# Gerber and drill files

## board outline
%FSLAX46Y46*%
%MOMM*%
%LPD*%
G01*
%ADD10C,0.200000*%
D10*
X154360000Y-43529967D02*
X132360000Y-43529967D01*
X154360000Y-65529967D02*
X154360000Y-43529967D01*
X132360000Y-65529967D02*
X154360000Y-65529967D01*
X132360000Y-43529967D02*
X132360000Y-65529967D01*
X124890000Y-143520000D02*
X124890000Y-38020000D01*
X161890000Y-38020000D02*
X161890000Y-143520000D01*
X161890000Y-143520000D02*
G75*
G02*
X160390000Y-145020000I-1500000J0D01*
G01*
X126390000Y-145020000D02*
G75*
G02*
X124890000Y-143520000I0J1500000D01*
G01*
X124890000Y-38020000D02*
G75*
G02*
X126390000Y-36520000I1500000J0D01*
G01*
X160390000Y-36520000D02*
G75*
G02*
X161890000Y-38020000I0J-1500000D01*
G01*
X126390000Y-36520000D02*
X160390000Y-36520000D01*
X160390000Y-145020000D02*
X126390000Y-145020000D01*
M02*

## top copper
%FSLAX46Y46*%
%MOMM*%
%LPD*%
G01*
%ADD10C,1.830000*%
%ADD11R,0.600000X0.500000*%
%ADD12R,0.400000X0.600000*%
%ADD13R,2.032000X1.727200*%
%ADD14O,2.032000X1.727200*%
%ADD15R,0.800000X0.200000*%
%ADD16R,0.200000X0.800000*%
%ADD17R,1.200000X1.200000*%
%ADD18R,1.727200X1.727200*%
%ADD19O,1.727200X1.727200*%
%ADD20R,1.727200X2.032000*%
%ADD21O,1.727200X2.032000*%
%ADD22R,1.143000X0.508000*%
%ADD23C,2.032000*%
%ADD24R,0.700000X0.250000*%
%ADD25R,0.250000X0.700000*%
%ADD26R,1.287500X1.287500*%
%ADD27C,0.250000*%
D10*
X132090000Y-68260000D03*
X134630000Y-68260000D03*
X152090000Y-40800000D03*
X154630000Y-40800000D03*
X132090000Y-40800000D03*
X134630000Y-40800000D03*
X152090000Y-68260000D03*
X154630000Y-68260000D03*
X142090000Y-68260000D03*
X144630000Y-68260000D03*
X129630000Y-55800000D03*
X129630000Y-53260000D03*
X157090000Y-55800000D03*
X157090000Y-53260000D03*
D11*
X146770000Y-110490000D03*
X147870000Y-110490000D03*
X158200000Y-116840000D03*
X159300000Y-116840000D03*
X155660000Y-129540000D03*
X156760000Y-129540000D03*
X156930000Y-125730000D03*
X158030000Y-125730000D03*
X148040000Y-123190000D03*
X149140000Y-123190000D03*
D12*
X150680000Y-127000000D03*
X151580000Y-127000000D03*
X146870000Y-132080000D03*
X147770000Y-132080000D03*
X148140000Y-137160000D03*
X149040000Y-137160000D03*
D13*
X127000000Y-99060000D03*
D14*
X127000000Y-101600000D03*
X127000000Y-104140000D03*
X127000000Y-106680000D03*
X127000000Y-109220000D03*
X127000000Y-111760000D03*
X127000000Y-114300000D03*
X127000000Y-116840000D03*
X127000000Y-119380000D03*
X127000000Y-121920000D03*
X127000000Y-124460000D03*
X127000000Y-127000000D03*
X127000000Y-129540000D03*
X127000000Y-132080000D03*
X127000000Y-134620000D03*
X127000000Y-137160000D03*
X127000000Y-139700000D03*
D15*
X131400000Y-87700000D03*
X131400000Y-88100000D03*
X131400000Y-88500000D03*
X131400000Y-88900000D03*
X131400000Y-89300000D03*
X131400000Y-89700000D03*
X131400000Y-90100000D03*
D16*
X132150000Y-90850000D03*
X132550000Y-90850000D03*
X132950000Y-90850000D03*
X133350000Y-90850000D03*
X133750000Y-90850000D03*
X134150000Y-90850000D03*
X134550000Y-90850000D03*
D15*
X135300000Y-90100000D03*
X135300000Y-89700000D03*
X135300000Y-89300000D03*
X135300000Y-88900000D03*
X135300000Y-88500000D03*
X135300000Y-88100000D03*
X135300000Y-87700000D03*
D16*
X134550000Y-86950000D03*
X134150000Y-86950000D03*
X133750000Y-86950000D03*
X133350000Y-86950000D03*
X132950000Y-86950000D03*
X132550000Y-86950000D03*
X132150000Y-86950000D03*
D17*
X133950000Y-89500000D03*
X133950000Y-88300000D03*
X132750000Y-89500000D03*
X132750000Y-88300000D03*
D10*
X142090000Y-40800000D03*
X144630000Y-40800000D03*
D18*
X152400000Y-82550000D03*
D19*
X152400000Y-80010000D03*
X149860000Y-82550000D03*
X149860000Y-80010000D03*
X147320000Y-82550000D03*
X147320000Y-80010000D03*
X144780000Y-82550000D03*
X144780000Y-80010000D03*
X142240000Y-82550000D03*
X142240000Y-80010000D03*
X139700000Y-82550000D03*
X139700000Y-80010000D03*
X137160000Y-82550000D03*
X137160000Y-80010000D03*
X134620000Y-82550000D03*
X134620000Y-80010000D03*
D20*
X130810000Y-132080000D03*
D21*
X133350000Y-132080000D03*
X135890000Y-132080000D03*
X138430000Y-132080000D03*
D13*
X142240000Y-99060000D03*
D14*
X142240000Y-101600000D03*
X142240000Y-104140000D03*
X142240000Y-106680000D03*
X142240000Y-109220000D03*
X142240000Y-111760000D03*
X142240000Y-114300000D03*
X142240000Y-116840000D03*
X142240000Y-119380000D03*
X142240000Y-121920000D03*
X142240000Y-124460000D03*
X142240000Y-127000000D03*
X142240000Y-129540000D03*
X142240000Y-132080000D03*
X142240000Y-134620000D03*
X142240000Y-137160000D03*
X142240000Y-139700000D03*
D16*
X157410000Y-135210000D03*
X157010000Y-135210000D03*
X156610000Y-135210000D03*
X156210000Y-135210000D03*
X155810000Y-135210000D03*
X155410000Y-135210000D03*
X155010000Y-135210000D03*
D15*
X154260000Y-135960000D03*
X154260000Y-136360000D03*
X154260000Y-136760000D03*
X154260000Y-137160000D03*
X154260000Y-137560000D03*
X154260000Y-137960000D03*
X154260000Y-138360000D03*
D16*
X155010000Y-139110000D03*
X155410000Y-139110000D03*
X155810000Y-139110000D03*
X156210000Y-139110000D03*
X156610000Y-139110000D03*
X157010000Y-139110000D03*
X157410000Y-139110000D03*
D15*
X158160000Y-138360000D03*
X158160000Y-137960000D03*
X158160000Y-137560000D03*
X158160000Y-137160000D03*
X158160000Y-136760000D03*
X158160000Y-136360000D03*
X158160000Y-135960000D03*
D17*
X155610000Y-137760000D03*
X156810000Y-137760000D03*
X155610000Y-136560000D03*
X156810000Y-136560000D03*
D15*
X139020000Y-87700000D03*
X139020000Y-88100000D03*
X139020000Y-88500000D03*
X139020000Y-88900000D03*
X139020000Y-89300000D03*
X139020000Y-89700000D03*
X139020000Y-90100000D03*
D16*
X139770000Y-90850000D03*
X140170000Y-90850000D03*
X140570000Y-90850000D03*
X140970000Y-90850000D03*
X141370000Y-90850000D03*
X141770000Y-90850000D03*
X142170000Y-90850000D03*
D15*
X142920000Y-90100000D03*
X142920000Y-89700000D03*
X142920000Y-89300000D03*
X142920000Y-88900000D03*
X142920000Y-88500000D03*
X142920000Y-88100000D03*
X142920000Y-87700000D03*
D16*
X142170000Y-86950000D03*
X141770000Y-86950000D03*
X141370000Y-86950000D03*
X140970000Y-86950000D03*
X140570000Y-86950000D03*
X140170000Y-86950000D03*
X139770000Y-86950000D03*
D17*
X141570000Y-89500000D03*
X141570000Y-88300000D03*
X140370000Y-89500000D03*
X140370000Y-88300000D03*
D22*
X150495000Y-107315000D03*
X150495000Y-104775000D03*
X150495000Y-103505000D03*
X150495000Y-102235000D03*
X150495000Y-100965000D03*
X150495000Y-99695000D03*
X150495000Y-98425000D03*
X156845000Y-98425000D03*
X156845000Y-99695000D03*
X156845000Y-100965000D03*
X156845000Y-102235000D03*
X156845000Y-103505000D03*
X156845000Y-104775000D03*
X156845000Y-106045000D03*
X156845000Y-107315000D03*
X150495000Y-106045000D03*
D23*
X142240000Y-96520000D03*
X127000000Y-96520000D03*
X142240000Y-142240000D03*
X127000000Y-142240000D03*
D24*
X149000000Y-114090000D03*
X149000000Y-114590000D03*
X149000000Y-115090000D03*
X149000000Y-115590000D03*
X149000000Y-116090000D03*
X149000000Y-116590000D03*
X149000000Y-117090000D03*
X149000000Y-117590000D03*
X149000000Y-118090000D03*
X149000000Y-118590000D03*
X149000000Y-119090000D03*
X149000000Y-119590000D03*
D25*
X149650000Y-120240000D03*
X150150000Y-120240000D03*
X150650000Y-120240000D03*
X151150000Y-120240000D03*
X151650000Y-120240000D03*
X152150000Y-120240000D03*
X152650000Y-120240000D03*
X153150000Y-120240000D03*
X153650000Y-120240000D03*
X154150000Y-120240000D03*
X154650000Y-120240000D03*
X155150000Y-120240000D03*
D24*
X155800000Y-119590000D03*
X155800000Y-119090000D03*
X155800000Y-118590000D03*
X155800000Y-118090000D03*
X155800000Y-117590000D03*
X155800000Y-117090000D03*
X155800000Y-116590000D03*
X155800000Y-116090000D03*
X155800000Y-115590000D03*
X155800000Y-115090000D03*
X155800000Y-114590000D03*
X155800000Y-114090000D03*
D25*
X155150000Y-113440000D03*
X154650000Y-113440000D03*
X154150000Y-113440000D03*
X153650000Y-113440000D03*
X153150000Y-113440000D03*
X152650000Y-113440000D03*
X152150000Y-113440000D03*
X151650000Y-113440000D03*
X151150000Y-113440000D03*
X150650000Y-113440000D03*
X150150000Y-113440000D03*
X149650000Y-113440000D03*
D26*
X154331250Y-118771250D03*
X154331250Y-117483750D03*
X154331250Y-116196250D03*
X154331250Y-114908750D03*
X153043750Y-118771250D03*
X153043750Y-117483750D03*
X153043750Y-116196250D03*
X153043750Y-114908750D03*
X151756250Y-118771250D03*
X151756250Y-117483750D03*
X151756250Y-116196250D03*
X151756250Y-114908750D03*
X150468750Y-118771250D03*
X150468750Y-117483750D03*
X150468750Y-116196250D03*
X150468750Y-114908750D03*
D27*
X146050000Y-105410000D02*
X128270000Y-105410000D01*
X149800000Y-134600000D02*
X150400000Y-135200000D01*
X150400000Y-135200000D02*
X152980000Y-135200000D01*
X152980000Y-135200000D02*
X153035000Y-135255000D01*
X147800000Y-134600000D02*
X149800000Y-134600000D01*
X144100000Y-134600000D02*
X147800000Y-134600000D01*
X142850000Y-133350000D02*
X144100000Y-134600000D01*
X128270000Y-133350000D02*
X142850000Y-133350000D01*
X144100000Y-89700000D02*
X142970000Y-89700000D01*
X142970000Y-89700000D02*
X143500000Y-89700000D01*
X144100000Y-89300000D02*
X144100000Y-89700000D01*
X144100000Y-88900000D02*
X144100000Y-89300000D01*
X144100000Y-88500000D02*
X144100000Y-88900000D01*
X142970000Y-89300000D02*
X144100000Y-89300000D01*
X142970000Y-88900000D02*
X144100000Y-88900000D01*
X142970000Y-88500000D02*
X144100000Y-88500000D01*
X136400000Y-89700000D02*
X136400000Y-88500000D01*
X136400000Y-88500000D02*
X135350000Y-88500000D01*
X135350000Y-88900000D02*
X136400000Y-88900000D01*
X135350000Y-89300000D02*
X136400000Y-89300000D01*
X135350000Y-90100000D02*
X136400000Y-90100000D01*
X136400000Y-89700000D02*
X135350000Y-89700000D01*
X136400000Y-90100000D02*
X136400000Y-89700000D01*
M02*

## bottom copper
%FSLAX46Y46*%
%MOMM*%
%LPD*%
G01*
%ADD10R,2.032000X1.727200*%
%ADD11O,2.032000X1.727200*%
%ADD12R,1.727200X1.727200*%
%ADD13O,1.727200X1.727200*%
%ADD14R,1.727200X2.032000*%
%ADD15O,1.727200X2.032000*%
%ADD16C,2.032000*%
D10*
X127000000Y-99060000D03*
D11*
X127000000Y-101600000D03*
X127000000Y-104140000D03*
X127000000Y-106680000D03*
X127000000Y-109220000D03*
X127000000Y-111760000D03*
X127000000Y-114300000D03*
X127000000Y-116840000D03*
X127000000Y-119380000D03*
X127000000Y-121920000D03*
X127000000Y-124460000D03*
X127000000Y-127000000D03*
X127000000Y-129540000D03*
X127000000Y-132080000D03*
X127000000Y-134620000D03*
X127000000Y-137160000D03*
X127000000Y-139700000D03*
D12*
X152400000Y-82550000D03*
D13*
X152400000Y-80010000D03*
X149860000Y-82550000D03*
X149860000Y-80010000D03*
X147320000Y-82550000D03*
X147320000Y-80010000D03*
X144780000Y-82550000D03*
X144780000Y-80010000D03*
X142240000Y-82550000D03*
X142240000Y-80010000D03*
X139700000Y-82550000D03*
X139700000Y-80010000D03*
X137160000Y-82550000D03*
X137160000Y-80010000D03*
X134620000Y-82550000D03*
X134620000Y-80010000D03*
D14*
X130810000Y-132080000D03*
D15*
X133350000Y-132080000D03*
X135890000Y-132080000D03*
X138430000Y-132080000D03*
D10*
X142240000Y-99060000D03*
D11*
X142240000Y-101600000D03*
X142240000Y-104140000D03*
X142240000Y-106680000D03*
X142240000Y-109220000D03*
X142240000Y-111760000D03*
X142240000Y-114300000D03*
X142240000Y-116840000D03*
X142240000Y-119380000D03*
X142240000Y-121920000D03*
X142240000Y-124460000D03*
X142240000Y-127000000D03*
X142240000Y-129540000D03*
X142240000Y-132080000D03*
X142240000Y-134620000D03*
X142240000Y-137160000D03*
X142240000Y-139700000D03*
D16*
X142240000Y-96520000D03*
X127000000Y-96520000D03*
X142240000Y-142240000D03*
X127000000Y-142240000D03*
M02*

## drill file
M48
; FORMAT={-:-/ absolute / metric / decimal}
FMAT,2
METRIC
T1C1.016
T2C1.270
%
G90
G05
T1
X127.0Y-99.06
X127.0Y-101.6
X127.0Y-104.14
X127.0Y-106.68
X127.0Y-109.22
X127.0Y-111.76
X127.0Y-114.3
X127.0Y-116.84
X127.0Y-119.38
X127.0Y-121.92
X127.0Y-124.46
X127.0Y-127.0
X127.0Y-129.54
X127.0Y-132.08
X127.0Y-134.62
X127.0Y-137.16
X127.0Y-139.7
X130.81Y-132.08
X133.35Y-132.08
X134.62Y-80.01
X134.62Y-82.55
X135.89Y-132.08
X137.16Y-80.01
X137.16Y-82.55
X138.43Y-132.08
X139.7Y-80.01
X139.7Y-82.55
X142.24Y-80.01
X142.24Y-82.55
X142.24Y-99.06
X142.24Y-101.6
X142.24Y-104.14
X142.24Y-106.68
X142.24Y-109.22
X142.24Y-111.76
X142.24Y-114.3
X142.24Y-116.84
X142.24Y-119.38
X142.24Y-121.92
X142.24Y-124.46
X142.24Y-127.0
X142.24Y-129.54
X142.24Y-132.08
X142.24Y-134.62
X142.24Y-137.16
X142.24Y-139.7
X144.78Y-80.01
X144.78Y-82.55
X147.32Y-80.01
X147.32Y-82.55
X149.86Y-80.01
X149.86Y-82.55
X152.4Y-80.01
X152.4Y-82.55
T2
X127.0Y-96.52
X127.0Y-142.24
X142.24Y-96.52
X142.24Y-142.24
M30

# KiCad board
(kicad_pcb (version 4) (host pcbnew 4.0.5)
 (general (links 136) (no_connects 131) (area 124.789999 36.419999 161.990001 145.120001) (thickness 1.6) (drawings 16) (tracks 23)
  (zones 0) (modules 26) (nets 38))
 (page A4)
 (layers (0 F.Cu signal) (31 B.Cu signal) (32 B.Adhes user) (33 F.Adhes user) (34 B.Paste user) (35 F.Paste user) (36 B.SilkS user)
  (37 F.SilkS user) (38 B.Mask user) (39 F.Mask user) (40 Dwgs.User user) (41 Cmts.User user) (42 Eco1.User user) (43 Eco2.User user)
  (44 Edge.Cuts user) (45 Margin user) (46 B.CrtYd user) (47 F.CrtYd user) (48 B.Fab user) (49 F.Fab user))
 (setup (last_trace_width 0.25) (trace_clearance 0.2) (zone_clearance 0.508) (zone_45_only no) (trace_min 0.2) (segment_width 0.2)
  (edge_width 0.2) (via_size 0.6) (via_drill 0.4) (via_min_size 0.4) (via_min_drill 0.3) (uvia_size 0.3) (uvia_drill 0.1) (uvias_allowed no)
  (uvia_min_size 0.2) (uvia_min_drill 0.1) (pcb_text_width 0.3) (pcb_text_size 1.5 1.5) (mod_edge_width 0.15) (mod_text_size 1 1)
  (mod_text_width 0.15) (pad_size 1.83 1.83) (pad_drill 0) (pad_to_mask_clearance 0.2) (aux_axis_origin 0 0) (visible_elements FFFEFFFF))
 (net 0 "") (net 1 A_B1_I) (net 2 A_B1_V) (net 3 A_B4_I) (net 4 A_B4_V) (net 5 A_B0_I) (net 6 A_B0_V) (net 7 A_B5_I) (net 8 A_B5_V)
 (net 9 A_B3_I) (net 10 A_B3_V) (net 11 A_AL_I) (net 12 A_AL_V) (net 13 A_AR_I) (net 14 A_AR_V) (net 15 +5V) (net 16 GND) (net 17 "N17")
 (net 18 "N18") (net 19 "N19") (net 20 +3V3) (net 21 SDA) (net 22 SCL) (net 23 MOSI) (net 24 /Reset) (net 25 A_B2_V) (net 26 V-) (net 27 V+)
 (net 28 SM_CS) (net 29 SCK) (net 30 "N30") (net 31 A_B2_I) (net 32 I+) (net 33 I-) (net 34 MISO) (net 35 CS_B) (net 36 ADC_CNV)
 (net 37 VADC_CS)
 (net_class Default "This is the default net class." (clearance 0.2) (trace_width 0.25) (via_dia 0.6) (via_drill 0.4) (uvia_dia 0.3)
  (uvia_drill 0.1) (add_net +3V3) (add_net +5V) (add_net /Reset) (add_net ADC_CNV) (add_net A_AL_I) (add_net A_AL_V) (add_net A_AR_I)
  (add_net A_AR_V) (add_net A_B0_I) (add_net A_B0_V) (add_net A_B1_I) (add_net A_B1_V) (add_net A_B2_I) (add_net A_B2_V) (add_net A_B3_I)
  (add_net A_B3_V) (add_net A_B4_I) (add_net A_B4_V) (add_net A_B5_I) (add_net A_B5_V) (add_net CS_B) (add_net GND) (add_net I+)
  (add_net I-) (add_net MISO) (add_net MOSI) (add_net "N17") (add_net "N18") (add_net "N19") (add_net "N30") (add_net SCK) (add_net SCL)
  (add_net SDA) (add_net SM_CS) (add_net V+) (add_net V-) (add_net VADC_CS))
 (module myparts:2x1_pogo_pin (layer F.Cu) (at 132.09 68.26)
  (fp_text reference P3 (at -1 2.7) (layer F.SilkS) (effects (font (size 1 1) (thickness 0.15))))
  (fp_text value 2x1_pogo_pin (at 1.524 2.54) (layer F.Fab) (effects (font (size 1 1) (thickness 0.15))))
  (pad 1 smd circle (at 0 0) (size 1.83 1.83) (layers F.Cu F.Paste F.Mask) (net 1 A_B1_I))
  (pad 2 smd circle (at 2.54 0) (size 1.83 1.83) (layers F.Cu F.Paste F.Mask) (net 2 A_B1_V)))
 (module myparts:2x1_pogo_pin (layer F.Cu) (at 152.09 40.8)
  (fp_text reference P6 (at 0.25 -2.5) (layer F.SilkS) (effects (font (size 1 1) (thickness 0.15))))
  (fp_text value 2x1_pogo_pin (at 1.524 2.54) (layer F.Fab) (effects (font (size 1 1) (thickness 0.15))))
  (pad 1 smd circle (at 0 0) (size 1.83 1.83) (layers F.Cu F.Paste F.Mask) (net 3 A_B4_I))
  (pad 2 smd circle (at 2.54 0) (size 1.83 1.83) (layers F.Cu F.Paste F.Mask) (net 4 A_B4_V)))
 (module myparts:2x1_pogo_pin (layer F.Cu) (at 132.09 40.8)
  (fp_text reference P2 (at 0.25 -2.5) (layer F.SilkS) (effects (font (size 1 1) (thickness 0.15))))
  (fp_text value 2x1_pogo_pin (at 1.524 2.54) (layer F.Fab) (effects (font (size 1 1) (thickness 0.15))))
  (pad 1 smd circle (at 0 0) (size 1.83 1.83) (layers F.Cu F.Paste F.Mask) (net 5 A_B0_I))
  (pad 2 smd circle (at 2.54 0) (size 1.83 1.83) (layers F.Cu F.Paste F.Mask) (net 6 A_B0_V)))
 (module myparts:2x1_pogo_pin (layer F.Cu) (at 152.09 68.26)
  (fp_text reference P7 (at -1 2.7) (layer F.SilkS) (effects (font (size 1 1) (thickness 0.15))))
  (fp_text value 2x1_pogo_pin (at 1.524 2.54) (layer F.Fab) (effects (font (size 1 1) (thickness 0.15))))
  (pad 1 smd circle (at 0 0) (size 1.83 1.83) (layers F.Cu F.Paste F.Mask) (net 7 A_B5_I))
  (pad 2 smd circle (at 2.54 0) (size 1.83 1.83) (layers F.Cu F.Paste F.Mask) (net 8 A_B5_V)))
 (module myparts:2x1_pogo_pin (layer F.Cu) (at 142.09 68.26)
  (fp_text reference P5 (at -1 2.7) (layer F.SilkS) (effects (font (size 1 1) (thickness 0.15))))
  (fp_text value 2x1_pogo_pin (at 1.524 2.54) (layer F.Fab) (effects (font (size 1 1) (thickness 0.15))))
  (pad 1 smd circle (at 0 0) (size 1.83 1.83) (layers F.Cu F.Paste F.Mask) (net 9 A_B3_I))
  (pad 2 smd circle (at 2.54 0) (size 1.83 1.83) (layers F.Cu F.Paste F.Mask) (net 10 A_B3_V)))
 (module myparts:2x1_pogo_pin (layer F.Cu) (at 129.63 55.8 90)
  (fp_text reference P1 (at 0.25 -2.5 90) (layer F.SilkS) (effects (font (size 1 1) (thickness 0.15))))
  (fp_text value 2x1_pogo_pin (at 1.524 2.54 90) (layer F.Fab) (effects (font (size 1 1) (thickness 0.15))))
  (pad 1 smd circle (at 0 0 90) (size 1.83 1.83) (layers F.Cu F.Paste F.Mask) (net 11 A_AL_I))
  (pad 2 smd circle (at 2.54 0 90) (size 1.83 1.83) (layers F.Cu F.Paste F.Mask) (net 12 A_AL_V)))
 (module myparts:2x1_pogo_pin (layer F.Cu) (at 157.09 55.8 90)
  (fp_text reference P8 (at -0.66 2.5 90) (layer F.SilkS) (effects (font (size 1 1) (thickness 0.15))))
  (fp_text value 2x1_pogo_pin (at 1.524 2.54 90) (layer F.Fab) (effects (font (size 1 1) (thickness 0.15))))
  (pad 1 smd circle (at 0 0 90) (size 1.83 1.83) (layers F.Cu F.Paste F.Mask) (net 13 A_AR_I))
  (pad 2 smd circle (at 2.54 0 90) (size 1.83 1.83) (layers F.Cu F.Paste F.Mask) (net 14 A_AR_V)))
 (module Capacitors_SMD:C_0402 (layer F.Cu) (at 147.32 110.49)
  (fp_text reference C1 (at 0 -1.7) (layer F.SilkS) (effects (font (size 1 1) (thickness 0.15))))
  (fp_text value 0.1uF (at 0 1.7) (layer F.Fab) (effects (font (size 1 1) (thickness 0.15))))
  (pad 1 smd rect (at -0.55 0) (size 0.6 0.5) (layers F.Cu F.Paste F.Mask) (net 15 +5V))
  (pad 2 smd rect (at 0.55 0) (size 0.6 0.5) (layers F.Cu F.Paste F.Mask) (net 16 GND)))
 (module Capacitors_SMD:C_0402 (layer F.Cu) (at 158.75 116.84)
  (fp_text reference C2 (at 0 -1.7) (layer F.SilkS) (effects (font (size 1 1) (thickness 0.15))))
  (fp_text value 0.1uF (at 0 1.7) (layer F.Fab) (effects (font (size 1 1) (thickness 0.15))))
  (pad 1 smd rect (at -0.55 0) (size 0.6 0.5) (layers F.Cu F.Paste F.Mask) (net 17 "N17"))
  (pad 2 smd rect (at 0.55 0) (size 0.6 0.5) (layers F.Cu F.Paste F.Mask) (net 16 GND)))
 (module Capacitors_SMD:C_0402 (layer F.Cu) (at 156.21 129.54)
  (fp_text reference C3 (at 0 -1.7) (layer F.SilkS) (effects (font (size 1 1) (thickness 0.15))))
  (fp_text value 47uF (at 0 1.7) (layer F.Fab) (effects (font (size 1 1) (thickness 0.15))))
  (pad 1 smd rect (at -0.55 0) (size 0.6 0.5) (layers F.Cu F.Paste F.Mask) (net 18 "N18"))
  (pad 2 smd rect (at 0.55 0) (size 0.6 0.5) (layers F.Cu F.Paste F.Mask) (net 16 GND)))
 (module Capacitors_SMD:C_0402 (layer F.Cu) (at 157.48 125.73)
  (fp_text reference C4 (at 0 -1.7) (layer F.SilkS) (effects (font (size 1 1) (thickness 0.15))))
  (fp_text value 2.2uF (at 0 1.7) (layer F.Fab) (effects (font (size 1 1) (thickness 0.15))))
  (pad 1 smd rect (at -0.55 0) (size 0.6 0.5) (layers F.Cu F.Paste F.Mask) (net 16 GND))
  (pad 2 smd rect (at 0.55 0) (size 0.6 0.5) (layers F.Cu F.Paste F.Mask) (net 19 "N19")))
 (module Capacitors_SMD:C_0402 (layer F.Cu) (at 148.59 123.19)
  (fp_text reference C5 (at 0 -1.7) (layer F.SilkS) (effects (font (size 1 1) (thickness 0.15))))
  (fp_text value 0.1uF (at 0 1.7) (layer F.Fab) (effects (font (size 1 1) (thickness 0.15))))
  (pad 1 smd rect (at -0.55 0) (size 0.6 0.5) (layers F.Cu F.Paste F.Mask) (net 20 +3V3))
  (pad 2 smd rect (at 0.55 0) (size 0.6 0.5) (layers F.Cu F.Paste F.Mask) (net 16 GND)))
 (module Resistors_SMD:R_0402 (layer F.Cu) (at 151.13 127)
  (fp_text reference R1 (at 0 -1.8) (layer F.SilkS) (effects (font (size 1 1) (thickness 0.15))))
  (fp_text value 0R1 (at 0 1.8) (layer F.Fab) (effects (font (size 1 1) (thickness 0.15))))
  (pad 1 smd rect (at -0.45 0) (size 0.4 0.6) (layers F.Cu F.Paste F.Mask))
  (pad 2 smd rect (at 0.45 0) (size 0.4 0.6) (layers F.Cu F.Paste F.Mask) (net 16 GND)))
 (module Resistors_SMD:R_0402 (layer F.Cu) (at 147.32 132.08)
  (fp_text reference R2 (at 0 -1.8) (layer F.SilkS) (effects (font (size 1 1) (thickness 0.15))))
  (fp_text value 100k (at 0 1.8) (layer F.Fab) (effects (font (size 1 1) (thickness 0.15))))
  (pad 1 smd rect (at -0.45 0) (size 0.4 0.6) (layers F.Cu F.Paste F.Mask) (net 20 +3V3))
  (pad 2 smd rect (at 0.45 0) (size 0.4 0.6) (layers F.Cu F.Paste F.Mask) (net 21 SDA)))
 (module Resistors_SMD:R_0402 (layer F.Cu) (at 148.59 137.16)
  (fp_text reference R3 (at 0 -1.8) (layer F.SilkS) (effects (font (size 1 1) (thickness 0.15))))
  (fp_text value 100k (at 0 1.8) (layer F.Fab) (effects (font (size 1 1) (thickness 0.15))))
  (pad 1 smd rect (at -0.45 0) (size 0.4 0.6) (layers F.Cu F.Paste F.Mask) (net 20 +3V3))
  (pad 2 smd rect (at 0.45 0) (size 0.4 0.6) (layers F.Cu F.Paste F.Mask) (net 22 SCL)))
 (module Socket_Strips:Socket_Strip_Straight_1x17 (layer F.Cu) (at 127 99.06 270)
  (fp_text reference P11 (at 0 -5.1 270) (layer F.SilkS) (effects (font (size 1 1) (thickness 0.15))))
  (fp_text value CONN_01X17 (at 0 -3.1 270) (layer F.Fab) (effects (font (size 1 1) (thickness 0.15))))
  (pad 1 thru_hole rect (at 0 0 270) (size 1.7272 2.032) (drill 1.016) (layers *.Cu *.Mask) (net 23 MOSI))
  (pad 2 thru_hole oval (at 2.54 0 270) (size 1.7272 2.032) (drill 1.016) (layers *.Cu *.Mask))
  (pad 3 thru_hole oval (at 5.08 0 270) (size 1.7272 2.032) (drill 1.016) (layers *.Cu *.Mask))
  (pad 4 thru_hole oval (at 7.62 0 270) (size 1.7272 2.032) (drill 1.016) (layers *.Cu *.Mask))
  (pad 5 thru_hole oval (at 10.16 0 270) (size 1.7272 2.032) (drill 1.016) (layers *.Cu *.Mask) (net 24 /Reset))
  (pad 6 thru_hole oval (at 12.7 0 270) (size 1.7272 2.032) (drill 1.016) (layers *.Cu *.Mask) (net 16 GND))
  (pad 7 thru_hole oval (at 15.24 0 270) (size 1.7272 2.032) (drill 1.016) (layers *.Cu *.Mask) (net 21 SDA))
  (pad 8 thru_hole oval (at 17.78 0 270) (size 1.7272 2.032) (drill 1.016) (layers *.Cu *.Mask) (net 22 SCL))
  (pad 9 thru_hole oval (at 20.32 0 270) (size 1.7272 2.032) (drill 1.016) (layers *.Cu *.Mask))
  (pad 10 thru_hole oval (at 22.86 0 270) (size 1.7272 2.032) (drill 1.016) (layers *.Cu *.Mask))
  (pad 11 thru_hole oval (at 25.4 0 270) (size 1.7272 2.032) (drill 1.016) (layers *.Cu *.Mask))
  (pad 12 thru_hole oval (at 27.94 0 270) (size 1.7272 2.032) (drill 1.016) (layers *.Cu *.Mask))
  (pad 13 thru_hole oval (at 30.48 0 270) (size 1.7272 2.032) (drill 1.016) (layers *.Cu *.Mask))
  (pad 14 thru_hole oval (at 33.02 0 270) (size 1.7272 2.032) (drill 1.016) (layers *.Cu *.Mask))
  (pad 15 thru_hole oval (at 35.56 0 270) (size 1.7272 2.032) (drill 1.016) (layers *.Cu *.Mask))
  (pad 16 thru_hole oval (at 38.1 0 270) (size 1.7272 2.032) (drill 1.016) (layers *.Cu *.Mask))
  (pad 17 thru_hole oval (at 40.64 0 270) (size 1.7272 2.032) (drill 1.016) (layers *.Cu *.Mask)))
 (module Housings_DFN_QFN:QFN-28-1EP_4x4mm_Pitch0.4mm (layer F.Cu) (at 133.35 88.9)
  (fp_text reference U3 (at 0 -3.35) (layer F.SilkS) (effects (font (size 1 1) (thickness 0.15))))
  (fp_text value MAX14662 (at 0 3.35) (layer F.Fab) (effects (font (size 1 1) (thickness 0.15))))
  (pad 1 smd rect (at -1.95 -1.2) (size 0.8 0.2) (layers F.Cu F.Paste F.Mask) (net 20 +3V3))
  (pad 2 smd rect (at -1.95 -0.8) (size 0.8 0.2) (layers F.Cu F.Paste F.Mask) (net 12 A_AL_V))
  (pad 3 smd rect (at -1.95 -0.4) (size 0.8 0.2) (layers F.Cu F.Paste F.Mask) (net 6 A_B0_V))
  (pad 4 smd rect (at -1.95 0) (size 0.8 0.2) (layers F.Cu F.Paste F.Mask) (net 2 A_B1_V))
  (pad 5 smd rect (at -1.95 0.4) (size 0.8 0.2) (layers F.Cu F.Paste F.Mask) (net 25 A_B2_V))
  (pad 6 smd rect (at -1.95 0.8) (size 0.8 0.2) (layers F.Cu F.Paste F.Mask) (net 10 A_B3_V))
  (pad 7 smd rect (at -1.95 1.2) (size 0.8 0.2) (layers F.Cu F.Paste F.Mask) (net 4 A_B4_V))
  (pad 8 smd rect (at -1.2 1.95 90) (size 0.8 0.2) (layers F.Cu F.Paste F.Mask) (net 8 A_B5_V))
  (pad 9 smd rect (at -0.8 1.95 90) (size 0.8 0.2) (layers F.Cu F.Paste F.Mask) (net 14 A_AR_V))
  (pad 10 smd rect (at -0.4 1.95 90) (size 0.8 0.2) (layers F.Cu F.Paste F.Mask))
  (pad 11 smd rect (at 0 1.95 90) (size 0.8 0.2) (layers F.Cu F.Paste F.Mask) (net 16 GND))
  (pad 12 smd rect (at 0.4 1.95 90) (size 0.8 0.2) (layers F.Cu F.Paste F.Mask))
  (pad 13 smd rect (at 0.8 1.95 90) (size 0.8 0.2) (layers F.Cu F.Paste F.Mask))
  (pad 14 smd rect (at 1.2 1.95 90) (size 0.8 0.2) (layers F.Cu F.Paste F.Mask) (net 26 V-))
  (pad 15 smd rect (at 1.95 1.2) (size 0.8 0.2) (layers F.Cu F.Paste F.Mask) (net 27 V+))
  (pad 16 smd rect (at 1.95 0.8) (size 0.8 0.2) (layers F.Cu F.Paste F.Mask) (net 27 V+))
  (pad 17 smd rect (at 1.95 0.4) (size 0.8 0.2) (layers F.Cu F.Paste F.Mask) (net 27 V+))
  (pad 18 smd rect (at 1.95 0) (size 0.8 0.2) (layers F.Cu F.Paste F.Mask) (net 27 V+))
  (pad 19 smd rect (at 1.95 -0.4) (size 0.8 0.2) (layers F.Cu F.Paste F.Mask) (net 27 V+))
  (pad 20 smd rect (at 1.95 -0.8) (size 0.8 0.2) (layers F.Cu F.Paste F.Mask) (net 27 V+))
  (pad 21 smd rect (at 1.95 -1.2) (size 0.8 0.2) (layers F.Cu F.Paste F.Mask) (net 26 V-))
  (pad 22 smd rect (at 1.2 -1.95 90) (size 0.8 0.2) (layers F.Cu F.Paste F.Mask) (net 20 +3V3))
  (pad 23 smd rect (at 0.8 -1.95 90) (size 0.8 0.2) (layers F.Cu F.Paste F.Mask) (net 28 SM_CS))
  (pad 24 smd rect (at 0.4 -1.95 90) (size 0.8 0.2) (layers F.Cu F.Paste F.Mask) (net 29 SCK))
  (pad 25 smd rect (at 0 -1.95 90) (size 0.8 0.2) (layers F.Cu F.Paste F.Mask) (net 16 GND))
  (pad 26 smd rect (at -0.4 -1.95 90) (size 0.8 0.2) (layers F.Cu F.Paste F.Mask) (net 20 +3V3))
  (pad 27 smd rect (at -0.8 -1.95 90) (size 0.8 0.2) (layers F.Cu F.Paste F.Mask) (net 23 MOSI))
  (pad 28 smd rect (at -1.2 -1.95 90) (size 0.8 0.2) (layers F.Cu F.Paste F.Mask) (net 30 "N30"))
  (pad 29 smd rect (at 0.6 0.6) (size 1.2 1.2) (layers F.Cu F.Paste F.Mask) (solder_paste_margin_ratio -0.2))
  (pad 29 smd rect (at 0.6 -0.6) (size 1.2 1.2) (layers F.Cu F.Paste F.Mask) (solder_paste_margin_ratio -0.2))
  (pad 29 smd rect (at -0.6 0.6) (size 1.2 1.2) (layers F.Cu F.Paste F.Mask) (solder_paste_margin_ratio -0.2))
  (pad 29 smd rect (at -0.6 -0.6) (size 1.2 1.2) (layers F.Cu F.Paste F.Mask) (solder_paste_margin_ratio -0.2)))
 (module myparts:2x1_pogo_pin (layer F.Cu) (at 142.09 40.8)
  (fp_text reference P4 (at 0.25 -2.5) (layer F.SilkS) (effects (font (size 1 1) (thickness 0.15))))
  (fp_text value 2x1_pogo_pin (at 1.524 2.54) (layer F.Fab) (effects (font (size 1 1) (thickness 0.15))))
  (pad 1 smd circle (at 0 0) (size 1.83 1.83) (layers F.Cu F.Paste F.Mask) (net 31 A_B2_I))
  (pad 2 smd circle (at 2.54 0) (size 1.83 1.83) (layers F.Cu F.Paste F.Mask) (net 25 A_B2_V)))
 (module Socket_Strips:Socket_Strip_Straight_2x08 (layer F.Cu) (at 152.4 82.55 180)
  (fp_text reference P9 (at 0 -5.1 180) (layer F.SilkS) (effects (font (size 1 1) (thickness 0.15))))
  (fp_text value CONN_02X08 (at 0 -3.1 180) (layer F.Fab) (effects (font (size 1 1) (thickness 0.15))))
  (pad 1 thru_hole rect (at 0 0 180) (size 1.7272 1.7272) (drill 1.016) (layers *.Cu *.Mask) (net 11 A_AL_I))
  (pad 2 thru_hole oval (at 0 2.54 180) (size 1.7272 1.7272) (drill 1.016) (layers *.Cu *.Mask) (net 12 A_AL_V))
  (pad 3 thru_hole oval (at 2.54 0 180) (size 1.7272 1.7272) (drill 1.016) (layers *.Cu *.Mask) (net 5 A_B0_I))
  (pad 4 thru_hole oval (at 2.54 2.54 180) (size 1.7272 1.7272) (drill 1.016) (layers *.Cu *.Mask) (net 6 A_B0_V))
  (pad 5 thru_hole oval (at 5.08 0 180) (size 1.7272 1.7272) (drill 1.016) (layers *.Cu *.Mask) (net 1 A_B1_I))
  (pad 6 thru_hole oval (at 5.08 2.54 180) (size 1.7272 1.7272) (drill 1.016) (layers *.Cu *.Mask) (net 2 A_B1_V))
  (pad 7 thru_hole oval (at 7.62 0 180) (size 1.7272 1.7272) (drill 1.016) (layers *.Cu *.Mask) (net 31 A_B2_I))
  (pad 8 thru_hole oval (at 7.62 2.54 180) (size 1.7272 1.7272) (drill 1.016) (layers *.Cu *.Mask) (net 25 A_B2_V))
  (pad 9 thru_hole oval (at 10.16 0 180) (size 1.7272 1.7272) (drill 1.016) (layers *.Cu *.Mask) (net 9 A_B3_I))
  (pad 10 thru_hole oval (at 10.16 2.54 180) (size 1.7272 1.7272) (drill 1.016) (layers *.Cu *.Mask) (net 10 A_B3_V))
  (pad 11 thru_hole oval (at 12.7 0 180) (size 1.7272 1.7272) (drill 1.016) (layers *.Cu *.Mask) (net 3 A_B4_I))
  (pad 12 thru_hole oval (at 12.7 2.54 180) (size 1.7272 1.7272) (drill 1.016) (layers *.Cu *.Mask) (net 4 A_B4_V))
  (pad 13 thru_hole oval (at 15.24 0 180) (size 1.7272 1.7272) (drill 1.016) (layers *.Cu *.Mask) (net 7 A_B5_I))
  (pad 14 thru_hole oval (at 15.24 2.54 180) (size 1.7272 1.7272) (drill 1.016) (layers *.Cu *.Mask) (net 8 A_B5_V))
  (pad 15 thru_hole oval (at 17.78 0 180) (size 1.7272 1.7272) (drill 1.016) (layers *.Cu *.Mask) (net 13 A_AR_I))
  (pad 16 thru_hole oval (at 17.78 2.54 180) (size 1.7272 1.7272) (drill 1.016) (layers *.Cu *.Mask) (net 14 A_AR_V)))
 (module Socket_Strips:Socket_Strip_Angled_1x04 (layer F.Cu) (at 130.81 132.08)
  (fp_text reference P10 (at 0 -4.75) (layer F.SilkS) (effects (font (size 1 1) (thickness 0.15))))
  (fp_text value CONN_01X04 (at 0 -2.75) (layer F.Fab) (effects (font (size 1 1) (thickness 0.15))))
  (pad 1 thru_hole rect (at 0 0) (size 1.7272 2.032) (drill 1.016) (layers *.Cu *.Mask) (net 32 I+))
  (pad 2 thru_hole oval (at 2.54 0) (size 1.7272 2.032) (drill 1.016) (layers *.Cu *.Mask) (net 27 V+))
  (pad 3 thru_hole oval (at 5.08 0) (size 1.7272 2.032) (drill 1.016) (layers *.Cu *.Mask) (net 26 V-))
  (pad 4 thru_hole oval (at 7.62 0) (size 1.7272 2.032) (drill 1.016) (layers *.Cu *.Mask) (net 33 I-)))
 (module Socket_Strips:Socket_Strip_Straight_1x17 (layer F.Cu) (at 142.24 99.06 270)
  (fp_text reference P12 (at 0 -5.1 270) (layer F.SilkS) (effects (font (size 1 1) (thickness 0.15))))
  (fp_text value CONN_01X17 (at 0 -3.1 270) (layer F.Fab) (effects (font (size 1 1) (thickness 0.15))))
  (pad 1 thru_hole rect (at 0 0 270) (size 1.7272 2.032) (drill 1.016) (layers *.Cu *.Mask) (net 29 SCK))
  (pad 2 thru_hole oval (at 2.54 0 270) (size 1.7272 2.032) (drill 1.016) (layers *.Cu *.Mask) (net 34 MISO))
  (pad 3 thru_hole oval (at 5.08 0 270) (size 1.7272 2.032) (drill 1.016) (layers *.Cu *.Mask))
  (pad 4 thru_hole oval (at 7.62 0 270) (size 1.7272 2.032) (drill 1.016) (layers *.Cu *.Mask) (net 16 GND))
  (pad 5 thru_hole oval (at 10.16 0 270) (size 1.7272 2.032) (drill 1.016) (layers *.Cu *.Mask) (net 24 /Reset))
  (pad 6 thru_hole oval (at 12.7 0 270) (size 1.7272 2.032) (drill 1.016) (layers *.Cu *.Mask) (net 15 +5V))
  (pad 7 thru_hole oval (at 15.24 0 270) (size 1.7272 2.032) (drill 1.016) (layers *.Cu *.Mask))
  (pad 8 thru_hole oval (at 17.78 0 270) (size 1.7272 2.032) (drill 1.016) (layers *.Cu *.Mask))
  (pad 9 thru_hole oval (at 20.32 0 270) (size 1.7272 2.032) (drill 1.016) (layers *.Cu *.Mask))
  (pad 10 thru_hole oval (at 22.86 0 270) (size 1.7272 2.032) (drill 1.016) (layers *.Cu *.Mask))
  (pad 11 thru_hole oval (at 25.4 0 270) (size 1.7272 2.032) (drill 1.016) (layers *.Cu *.Mask))
  (pad 12 thru_hole oval (at 27.94 0 270) (size 1.7272 2.032) (drill 1.016) (layers *.Cu *.Mask))
  (pad 13 thru_hole oval (at 30.48 0 270) (size 1.7272 2.032) (drill 1.016) (layers *.Cu *.Mask))
  (pad 14 thru_hole oval (at 33.02 0 270) (size 1.7272 2.032) (drill 1.016) (layers *.Cu *.Mask))
  (pad 15 thru_hole oval (at 35.56 0 270) (size 1.7272 2.032) (drill 1.016) (layers *.Cu *.Mask))
  (pad 16 thru_hole oval (at 38.1 0 270) (size 1.7272 2.032) (drill 1.016) (layers *.Cu *.Mask) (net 20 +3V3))
  (pad 17 thru_hole oval (at 40.64 0 270) (size 1.7272 2.032) (drill 1.016) (layers *.Cu *.Mask)))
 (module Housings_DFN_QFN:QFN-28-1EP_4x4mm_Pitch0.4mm (layer F.Cu) (at 156.21 137.16 270)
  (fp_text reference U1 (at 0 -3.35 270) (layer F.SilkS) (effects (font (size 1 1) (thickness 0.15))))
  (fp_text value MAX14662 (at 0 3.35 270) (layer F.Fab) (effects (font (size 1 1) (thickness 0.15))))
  (pad 1 smd rect (at -1.95 -1.2 270) (size 0.8 0.2) (layers F.Cu F.Paste F.Mask) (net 20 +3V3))
  (pad 2 smd rect (at -1.95 -0.8 270) (size 0.8 0.2) (layers F.Cu F.Paste F.Mask) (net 32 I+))
  (pad 3 smd rect (at -1.95 -0.4 270) (size 0.8 0.2) (layers F.Cu F.Paste F.Mask) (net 27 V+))
  (pad 4 smd rect (at -1.95 0 270) (size 0.8 0.2) (layers F.Cu F.Paste F.Mask) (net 26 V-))
  (pad 5 smd rect (at -1.95 0.4 270) (size 0.8 0.2) (layers F.Cu F.Paste F.Mask) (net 33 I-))
  (pad 6 smd rect (at -1.95 0.8 270) (size 0.8 0.2) (layers F.Cu F.Paste F.Mask))
  (pad 7 smd rect (at -1.95 1.2 270) (size 0.8 0.2) (layers F.Cu F.Paste F.Mask))
  (pad 8 smd rect (at -1.2 1.95) (size 0.8 0.2) (layers F.Cu F.Paste F.Mask))
  (pad 9 smd rect (at -0.8 1.95) (size 0.8 0.2) (layers F.Cu F.Paste F.Mask))
  (pad 10 smd rect (at -0.4 1.95) (size 0.8 0.2) (layers F.Cu F.Paste F.Mask))
  (pad 11 smd rect (at 0 1.95) (size 0.8 0.2) (layers F.Cu F.Paste F.Mask) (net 16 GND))
  (pad 12 smd rect (at 0.4 1.95) (size 0.8 0.2) (layers F.Cu F.Paste F.Mask))
  (pad 13 smd rect (at 0.8 1.95) (size 0.8 0.2) (layers F.Cu F.Paste F.Mask))
  (pad 14 smd rect (at 1.2 1.95) (size 0.8 0.2) (layers F.Cu F.Paste F.Mask))
  (pad 15 smd rect (at 1.95 1.2 270) (size 0.8 0.2) (layers F.Cu F.Paste F.Mask))
  (pad 16 smd rect (at 1.95 0.8 270) (size 0.8 0.2) (layers F.Cu F.Paste F.Mask))
  (pad 17 smd rect (at 1.95 0.4 270) (size 0.8 0.2) (layers F.Cu F.Paste F.Mask))
  (pad 18 smd rect (at 1.95 0 270) (size 0.8 0.2) (layers F.Cu F.Paste F.Mask))
  (pad 19 smd rect (at 1.95 -0.4 270) (size 0.8 0.2) (layers F.Cu F.Paste F.Mask))
  (pad 20 smd rect (at 1.95 -0.8 270) (size 0.8 0.2) (layers F.Cu F.Paste F.Mask))
  (pad 21 smd rect (at 1.95 -1.2 270) (size 0.8 0.2) (layers F.Cu F.Paste F.Mask))
  (pad 22 smd rect (at 1.2 -1.95) (size 0.8 0.2) (layers F.Cu F.Paste F.Mask) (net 20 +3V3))
  (pad 23 smd rect (at 0.8 -1.95) (size 0.8 0.2) (layers F.Cu F.Paste F.Mask) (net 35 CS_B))
  (pad 24 smd rect (at 0.4 -1.95) (size 0.8 0.2) (layers F.Cu F.Paste F.Mask) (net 29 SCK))
  (pad 25 smd rect (at 0 -1.95) (size 0.8 0.2) (layers F.Cu F.Paste F.Mask) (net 16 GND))
  (pad 26 smd rect (at -0.4 -1.95) (size 0.8 0.2) (layers F.Cu F.Paste F.Mask) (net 20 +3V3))
  (pad 27 smd rect (at -0.8 -1.95) (size 0.8 0.2) (layers F.Cu F.Paste F.Mask) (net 23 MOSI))
  (pad 28 smd rect (at -1.2 -1.95) (size 0.8 0.2) (layers F.Cu F.Paste F.Mask))
  (pad 29 smd rect (at 0.6 0.6 270) (size 1.2 1.2) (layers F.Cu F.Paste F.Mask) (solder_paste_margin_ratio -0.2))
  (pad 29 smd rect (at 0.6 -0.6 270) (size 1.2 1.2) (layers F.Cu F.Paste F.Mask) (solder_paste_margin_ratio -0.2))
  (pad 29 smd rect (at -0.6 0.6 270) (size 1.2 1.2) (layers F.Cu F.Paste F.Mask) (solder_paste_margin_ratio -0.2))
  (pad 29 smd rect (at -0.6 -0.6 270) (size 1.2 1.2) (layers F.Cu F.Paste F.Mask) (solder_paste_margin_ratio -0.2)))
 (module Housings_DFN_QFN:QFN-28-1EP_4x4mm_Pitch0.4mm (layer F.Cu) (at 140.97 88.9)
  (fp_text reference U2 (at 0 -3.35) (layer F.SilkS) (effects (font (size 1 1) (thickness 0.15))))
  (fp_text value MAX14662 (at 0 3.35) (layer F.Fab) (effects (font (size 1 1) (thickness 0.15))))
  (pad 1 smd rect (at -1.95 -1.2) (size 0.8 0.2) (layers F.Cu F.Paste F.Mask) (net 20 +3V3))
  (pad 2 smd rect (at -1.95 -0.8) (size 0.8 0.2) (layers F.Cu F.Paste F.Mask) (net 11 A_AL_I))
  (pad 3 smd rect (at -1.95 -0.4) (size 0.8 0.2) (layers F.Cu F.Paste F.Mask) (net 5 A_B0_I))
  (pad 4 smd rect (at -1.95 0) (size 0.8 0.2) (layers F.Cu F.Paste F.Mask) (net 1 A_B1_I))
  (pad 5 smd rect (at -1.95 0.4) (size 0.8 0.2) (layers F.Cu F.Paste F.Mask) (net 31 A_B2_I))
  (pad 6 smd rect (at -1.95 0.8) (size 0.8 0.2) (layers F.Cu F.Paste F.Mask) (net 9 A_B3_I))
  (pad 7 smd rect (at -1.95 1.2) (size 0.8 0.2) (layers F.Cu F.Paste F.Mask) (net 3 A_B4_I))
  (pad 8 smd rect (at -1.2 1.95 90) (size 0.8 0.2) (layers F.Cu F.Paste F.Mask) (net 7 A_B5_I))
  (pad 9 smd rect (at -0.8 1.95 90) (size 0.8 0.2) (layers F.Cu F.Paste F.Mask) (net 13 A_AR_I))
  (pad 10 smd rect (at -0.4 1.95 90) (size 0.8 0.2) (layers F.Cu F.Paste F.Mask))
  (pad 11 smd rect (at 0 1.95 90) (size 0.8 0.2) (layers F.Cu F.Paste F.Mask) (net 16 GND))
  (pad 12 smd rect (at 0.4 1.95 90) (size 0.8 0.2) (layers F.Cu F.Paste F.Mask))
  (pad 13 smd rect (at 0.8 1.95 90) (size 0.8 0.2) (layers F.Cu F.Paste F.Mask))
  (pad 14 smd rect (at 1.2 1.95 90) (size 0.8 0.2) (layers F.Cu F.Paste F.Mask) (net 33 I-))
  (pad 15 smd rect (at 1.95 1.2) (size 0.8 0.2) (layers F.Cu F.Paste F.Mask) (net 32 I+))
  (pad 16 smd rect (at 1.95 0.8) (size 0.8 0.2) (layers F.Cu F.Paste F.Mask) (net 32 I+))
  (pad 17 smd rect (at 1.95 0.4) (size 0.8 0.2) (layers F.Cu F.Paste F.Mask) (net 32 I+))
  (pad 18 smd rect (at 1.95 0) (size 0.8 0.2) (layers F.Cu F.Paste F.Mask) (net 32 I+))
  (pad 19 smd rect (at 1.95 -0.4) (size 0.8 0.2) (layers F.Cu F.Paste F.Mask) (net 32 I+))
  (pad 20 smd rect (at 1.95 -0.8) (size 0.8 0.2) (layers F.Cu F.Paste F.Mask) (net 32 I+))
  (pad 21 smd rect (at 1.95 -1.2) (size 0.8 0.2) (layers F.Cu F.Paste F.Mask) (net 33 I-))
  (pad 22 smd rect (at 1.2 -1.95 90) (size 0.8 0.2) (layers F.Cu F.Paste F.Mask) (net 20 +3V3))
  (pad 23 smd rect (at 0.8 -1.95 90) (size 0.8 0.2) (layers F.Cu F.Paste F.Mask) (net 30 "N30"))
  (pad 24 smd rect (at 0.4 -1.95 90) (size 0.8 0.2) (layers F.Cu F.Paste F.Mask) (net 29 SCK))
  (pad 25 smd rect (at 0 -1.95 90) (size 0.8 0.2) (layers F.Cu F.Paste F.Mask) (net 16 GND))
  (pad 26 smd rect (at -0.4 -1.95 90) (size 0.8 0.2) (layers F.Cu F.Paste F.Mask) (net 20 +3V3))
  (pad 27 smd rect (at -0.8 -1.95 90) (size 0.8 0.2) (layers F.Cu F.Paste F.Mask) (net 23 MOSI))
  (pad 28 smd rect (at -1.2 -1.95 90) (size 0.8 0.2) (layers F.Cu F.Paste F.Mask))
  (pad 29 smd rect (at 0.6 0.6) (size 1.2 1.2) (layers F.Cu F.Paste F.Mask) (solder_paste_margin_ratio -0.2))
  (pad 29 smd rect (at 0.6 -0.6) (size 1.2 1.2) (layers F.Cu F.Paste F.Mask) (solder_paste_margin_ratio -0.2))
  (pad 29 smd rect (at -0.6 0.6) (size 1.2 1.2) (layers F.Cu F.Paste F.Mask) (solder_paste_margin_ratio -0.2))
  (pad 29 smd rect (at -0.6 -0.6) (size 1.2 1.2) (layers F.Cu F.Paste F.Mask) (solder_paste_margin_ratio -0.2)))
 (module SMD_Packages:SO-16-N (layer F.Cu) (at 153.67 102.87 90)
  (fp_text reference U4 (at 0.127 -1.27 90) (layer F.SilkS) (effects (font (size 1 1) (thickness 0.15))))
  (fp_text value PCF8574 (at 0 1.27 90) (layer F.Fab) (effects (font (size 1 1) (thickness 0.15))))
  (pad 16 smd rect (at -4.445 -3.175 90) (size 0.508 1.143) (layers F.Cu F.Paste F.Mask) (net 20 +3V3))
  (pad 14 smd rect (at -1.905 -3.175 90) (size 0.508 1.143) (layers F.Cu F.Paste F.Mask) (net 22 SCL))
  (pad 13 smd rect (at -0.635 -3.175 90) (size 0.508 1.143) (layers F.Cu F.Paste F.Mask))
  (pad 12 smd rect (at 0.635 -3.175 90) (size 0.508 1.143) (layers F.Cu F.Paste F.Mask))
  (pad 11 smd rect (at 1.905 -3.175 90) (size 0.508 1.143) (layers F.Cu F.Paste F.Mask))
  (pad 10 smd rect (at 3.175 -3.175 90) (size 0.508 1.143) (layers F.Cu F.Paste F.Mask))
  (pad 9 smd rect (at 4.445 -3.175 90) (size 0.508 1.143) (layers F.Cu F.Paste F.Mask))
  (pad 8 smd rect (at 4.445 3.175 90) (size 0.508 1.143) (layers F.Cu F.Paste F.Mask) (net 16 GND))
  (pad 7 smd rect (at 3.175 3.175 90) (size 0.508 1.143) (layers F.Cu F.Paste F.Mask) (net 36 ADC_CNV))
  (pad 6 smd rect (at 1.905 3.175 90) (size 0.508 1.143) (layers F.Cu F.Paste F.Mask) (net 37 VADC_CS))
  (pad 5 smd rect (at 0.635 3.175 90) (size 0.508 1.143) (layers F.Cu F.Paste F.Mask) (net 35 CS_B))
  (pad 4 smd rect (at -0.635 3.175 90) (size 0.508 1.143) (layers F.Cu F.Paste F.Mask) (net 28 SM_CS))
  (pad 3 smd rect (at -1.905 3.175 90) (size 0.508 1.143) (layers F.Cu F.Paste F.Mask) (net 20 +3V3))
  (pad 2 smd rect (at -3.175 3.175 90) (size 0.508 1.143) (layers F.Cu F.Paste F.Mask) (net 16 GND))
  (pad 1 smd rect (at -4.445 3.175 90) (size 0.508 1.143) (layers F.Cu F.Paste F.Mask) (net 20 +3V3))
  (pad 15 smd rect (at -3.175 -3.175 90) (size 0.508 1.143) (layers F.Cu F.Paste F.Mask) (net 21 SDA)))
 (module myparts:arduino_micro (layer F.Cu) (at 127 96.52)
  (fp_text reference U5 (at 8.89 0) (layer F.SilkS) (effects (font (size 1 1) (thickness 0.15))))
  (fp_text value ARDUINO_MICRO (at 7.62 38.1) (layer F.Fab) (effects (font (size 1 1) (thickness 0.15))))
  (pad 2 thru_hole circle (at 15.24 0 180) (size 2.032 2.032) (drill 1.27) (layers *.Cu *.Mask F.SilkS))
  (pad 1 thru_hole circle (at 0 0 180) (size 2.032 2.032) (drill 1.27) (layers *.Cu *.Mask F.SilkS))
  (pad 3 thru_hole circle (at 15.24 45.72 180) (size 2.032 2.032) (drill 1.27) (layers *.Cu *.Mask F.SilkS))
  (pad 4 thru_hole circle (at 0 45.72 180) (size 2.032 2.032) (drill 1.27) (layers *.Cu *.Mask F.SilkS)))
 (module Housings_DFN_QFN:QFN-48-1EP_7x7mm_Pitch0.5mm (layer F.Cu) (at 152.4 116.84)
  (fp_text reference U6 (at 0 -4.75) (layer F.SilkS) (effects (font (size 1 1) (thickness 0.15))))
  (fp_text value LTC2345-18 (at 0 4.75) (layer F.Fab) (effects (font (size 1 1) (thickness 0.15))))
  (pad 1 smd rect (at -3.4 -2.75) (size 0.7 0.25) (layers F.Cu F.Paste F.Mask))
  (pad 2 smd rect (at -3.4 -2.25) (size 0.7 0.25) (layers F.Cu F.Paste F.Mask))
  (pad 3 smd rect (at -3.4 -1.75) (size 0.7 0.25) (layers F.Cu F.Paste F.Mask))
  (pad 4 smd rect (at -3.4 -1.25) (size 0.7 0.25) (layers F.Cu F.Paste F.Mask))
  (pad 5 smd rect (at -3.4 -0.75) (size 0.7 0.25) (layers F.Cu F.Paste F.Mask))
  (pad 6 smd rect (at -3.4 -0.25) (size 0.7 0.25) (layers F.Cu F.Paste F.Mask))
  (pad 7 smd rect (at -3.4 0.25) (size 0.7 0.25) (layers F.Cu F.Paste F.Mask))
  (pad 8 smd rect (at -3.4 0.75) (size 0.7 0.25) (layers F.Cu F.Paste F.Mask))
  (pad 9 smd rect (at -3.4 1.25) (size 0.7 0.25) (layers F.Cu F.Paste F.Mask))
  (pad 10 smd rect (at -3.4 1.75) (size 0.7 0.25) (layers F.Cu F.Paste F.Mask))
  (pad 11 smd rect (at -3.4 2.25) (size 0.7 0.25) (layers F.Cu F.Paste F.Mask))
  (pad 12 smd rect (at -3.4 2.75) (size 0.7 0.25) (layers F.Cu F.Paste F.Mask))
  (pad 13 smd rect (at -2.75 3.4 90) (size 0.7 0.25) (layers F.Cu F.Paste F.Mask))
  (pad 14 smd rect (at -2.25 3.4 90) (size 0.7 0.25) (layers F.Cu F.Paste F.Mask))
  (pad 15 smd rect (at -1.75 3.4 90) (size 0.7 0.25) (layers F.Cu F.Paste F.Mask) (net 16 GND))
  (pad 16 smd rect (at -1.25 3.4 90) (size 0.7 0.25) (layers F.Cu F.Paste F.Mask) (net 16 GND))
  (pad 17 smd rect (at -0.75 3.4 90) (size 0.7 0.25) (layers F.Cu F.Paste F.Mask) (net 16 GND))
  (pad 18 smd rect (at -0.25 3.4 90) (size 0.7 0.25) (layers F.Cu F.Paste F.Mask) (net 16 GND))
  (pad 19 smd rect (at 0.25 3.4 90) (size 0.7 0.25) (layers F.Cu F.Paste F.Mask) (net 17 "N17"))
  (pad 20 smd rect (at 0.75 3.4 90) (size 0.7 0.25) (layers F.Cu F.Paste F.Mask) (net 16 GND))
  (pad 21 smd rect (at 1.25 3.4 90) (size 0.7 0.25) (layers F.Cu F.Paste F.Mask) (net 18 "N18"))
  (pad 22 smd rect (at 1.75 3.4 90) (size 0.7 0.25) (layers F.Cu F.Paste F.Mask) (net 16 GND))
  (pad 23 smd rect (at 2.25 3.4 90) (size 0.7 0.25) (layers F.Cu F.Paste F.Mask) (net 16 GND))
  (pad 24 smd rect (at 2.75 3.4 90) (size 0.7 0.25) (layers F.Cu F.Paste F.Mask) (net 36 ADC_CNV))
  (pad 25 smd rect (at 3.4 2.75) (size 0.7 0.25) (layers F.Cu F.Paste F.Mask) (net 34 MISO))
  (pad 26 smd rect (at 3.4 2.25) (size 0.7 0.25) (layers F.Cu F.Paste F.Mask))
  (pad 27 smd rect (at 3.4 1.75) (size 0.7 0.25) (layers F.Cu F.Paste F.Mask))
  (pad 28 smd rect (at 3.4 1.25) (size 0.7 0.25) (layers F.Cu F.Paste F.Mask))
  (pad 29 smd rect (at 3.4 0.75) (size 0.7 0.25) (layers F.Cu F.Paste F.Mask) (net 29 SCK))
  (pad 30 smd rect (at 3.4 0.25) (size 0.7 0.25) (layers F.Cu F.Paste F.Mask) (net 16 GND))
  (pad 31 smd rect (at 3.4 -0.25) (size 0.7 0.25) (layers F.Cu F.Paste F.Mask) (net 20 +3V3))
  (pad 32 smd rect (at 3.4 -0.75) (size 0.7 0.25) (layers F.Cu F.Paste F.Mask))
  (pad 33 smd rect (at 3.4 -1.25) (size 0.7 0.25) (layers F.Cu F.Paste F.Mask))
  (pad 34 smd rect (at 3.4 -1.75) (size 0.7 0.25) (layers F.Cu F.Paste F.Mask))
  (pad 35 smd rect (at 3.4 -2.25) (size 0.7 0.25) (layers F.Cu F.Paste F.Mask))
  (pad 36 smd rect (at 3.4 -2.75) (size 0.7 0.25) (layers F.Cu F.Paste F.Mask))
  (pad 37 smd rect (at 2.75 -3.4 90) (size 0.7 0.25) (layers F.Cu F.Paste F.Mask) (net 23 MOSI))
  (pad 38 smd rect (at 2.25 -3.4 90) (size 0.7 0.25) (layers F.Cu F.Paste F.Mask))
  (pad 39 smd rect (at 1.75 -3.4 90) (size 0.7 0.25) (layers F.Cu F.Paste F.Mask) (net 37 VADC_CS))
  (pad 40 smd rect (at 1.25 -3.4 90) (size 0.7 0.25) (layers F.Cu F.Paste F.Mask) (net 19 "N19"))
  (pad 41 smd rect (at 0.75 -3.4 90) (size 0.7 0.25) (layers F.Cu F.Paste F.Mask) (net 16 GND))
  (pad 42 smd rect (at 0.25 -3.4 90) (size 0.7 0.25) (layers F.Cu F.Paste F.Mask) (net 15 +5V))
  (pad 43 smd rect (at -0.25 -3.4 90) (size 0.7 0.25) (layers F.Cu F.Paste F.Mask) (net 15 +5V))
  (pad 44 smd rect (at -0.75 -3.4 90) (size 0.7 0.25) (layers F.Cu F.Paste F.Mask) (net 16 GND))
  (pad 45 smd rect (at -1.25 -3.4 90) (size 0.7 0.25) (layers F.Cu F.Paste F.Mask) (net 16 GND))
  (pad 46 smd rect (at -1.75 -3.4 90) (size 0.7 0.25) (layers F.Cu F.Paste F.Mask) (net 16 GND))
  (pad 47 smd rect (at -2.25 -3.4 90) (size 0.7 0.25) (layers F.Cu F.Paste F.Mask))
  (pad 48 smd rect (at -2.75 -3.4 90) (size 0.7 0.25) (layers F.Cu F.Paste F.Mask))
  (pad 49 smd rect (at 1.93125 1.93125) (size 1.2875 1.2875) (layers F.Cu F.Paste F.Mask) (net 16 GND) (solder_paste_margin_ratio -0.2))
  (pad 49 smd rect (at 1.93125 0.64375) (size 1.2875 1.2875) (layers F.Cu F.Paste F.Mask) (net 16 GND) (solder_paste_margin_ratio -0.2))
  (pad 49 smd rect (at 1.93125 -0.64375) (size 1.2875 1.2875) (layers F.Cu F.Paste F.Mask) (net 16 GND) (solder_paste_margin_ratio -0.2))
  (pad 49 smd rect (at 1.93125 -1.93125) (size 1.2875 1.2875) (layers F.Cu F.Paste F.Mask) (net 16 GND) (solder_paste_margin_ratio -0.2))
  (pad 49 smd rect (at 0.64375 1.93125) (size 1.2875 1.2875) (layers F.Cu F.Paste F.Mask) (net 16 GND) (solder_paste_margin_ratio -0.2))
  (pad 49 smd rect (at 0.64375 0.64375) (size 1.2875 1.2875) (layers F.Cu F.Paste F.Mask) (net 16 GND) (solder_paste_margin_ratio -0.2))
  (pad 49 smd rect (at 0.64375 -0.64375) (size 1.2875 1.2875) (layers F.Cu F.Paste F.Mask) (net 16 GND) (solder_paste_margin_ratio -0.2))
  (pad 49 smd rect (at 0.64375 -1.93125) (size 1.2875 1.2875) (layers F.Cu F.Paste F.Mask) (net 16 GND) (solder_paste_margin_ratio -0.2))
  (pad 49 smd rect (at -0.64375 1.93125) (size 1.2875 1.2875) (layers F.Cu F.Paste F.Mask) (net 16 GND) (solder_paste_margin_ratio -0.2))
  (pad 49 smd rect (at -0.64375 0.64375) (size 1.2875 1.2875) (layers F.Cu F.Paste F.Mask) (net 16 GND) (solder_paste_margin_ratio -0.2))
  (pad 49 smd rect (at -0.64375 -0.64375) (size 1.2875 1.2875) (layers F.Cu F.Paste F.Mask) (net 16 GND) (solder_paste_margin_ratio -0.2))
  (pad 49 smd rect (at -0.64375 -1.93125) (size 1.2875 1.2875) (layers F.Cu F.Paste F.Mask) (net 16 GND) (solder_paste_margin_ratio -0.2))
  (pad 49 smd rect (at -1.93125 1.93125) (size 1.2875 1.2875) (layers F.Cu F.Paste F.Mask) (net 16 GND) (solder_paste_margin_ratio -0.2))
  (pad 49 smd rect (at -1.93125 0.64375) (size 1.2875 1.2875) (layers F.Cu F.Paste F.Mask) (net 16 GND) (solder_paste_margin_ratio -0.2))
  (pad 49 smd rect (at -1.93125 -0.64375) (size 1.2875 1.2875) (layers F.Cu F.Paste F.Mask) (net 16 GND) (solder_paste_margin_ratio -0.2))
  (pad 49 smd rect (at -1.93125 -1.93125) (size 1.2875 1.2875) (layers F.Cu F.Paste F.Mask) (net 16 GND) (solder_paste_margin_ratio -0.2)))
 (gr_line (start 154.36 43.529967) (end 132.36 43.529967) (layer Edge.Cuts) (width 0.2))
 (gr_line (start 154.36 65.529967) (end 154.36 43.529967) (layer Edge.Cuts) (width 0.2))
 (gr_line (start 132.36 65.529967) (end 154.36 65.529967) (layer Edge.Cuts) (width 0.2))
 (gr_line (start 132.36 43.529967) (end 132.36 65.529967) (layer Edge.Cuts) (width 0.2))
 (gr_line (start 124.89 143.52) (end 124.89 38.02) (angle 90) (layer Edge.Cuts) (width 0.2))
 (gr_line (start 161.89 38.02) (end 161.89 143.52) (angle 90) (layer Edge.Cuts) (width 0.2))
 (gr_arc (start 160.39 143.52) (end 161.89 143.52) (angle 90) (layer Edge.Cuts) (width 0.2))
 (gr_arc (start 126.39 143.52) (end 126.39 145.02) (angle 90) (layer Edge.Cuts) (width 0.2))
 (gr_arc (start 126.39 38.02) (end 124.89 38.02) (angle 90) (layer Edge.Cuts) (width 0.2))
 (gr_arc (start 160.39 38.02) (end 160.39 36.52) (angle 90) (layer Edge.Cuts) (width 0.2))
 (gr_line (start 126.39 36.52) (end 160.39 36.52) (angle 90) (layer Edge.Cuts) (width 0.2))
 (gr_line (start 160.39 145.02) (end 126.39 145.02) (angle 90) (layer Edge.Cuts) (width 0.2))
 (segment (start 146.05 105.41) (end 128.27 105.41) (width 0.25) (layer F.Cu) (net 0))
 (segment (start 149.8 134.6) (end 150.4 135.2) (width 0.25) (layer F.Cu) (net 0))
 (segment (start 150.4 135.2) (end 152.98 135.2) (width 0.25) (layer F.Cu) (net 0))
 (segment (start 152.98 135.2) (end 153.035 135.255) (width 0.25) (layer F.Cu) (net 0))
 (segment (start 147.8 134.6) (end 149.8 134.6) (width 0.25) (layer F.Cu) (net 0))
 (segment (start 144.1 134.6) (end 147.8 134.6) (width 0.25) (layer F.Cu) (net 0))
 (segment (start 142.85 133.35) (end 144.1 134.6) (width 0.25) (layer F.Cu) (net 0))
 (segment (start 128.27 133.35) (end 142.85 133.35) (width 0.25) (layer F.Cu) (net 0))
 (segment (start 144.1 89.7) (end 142.97 89.7) (width 0.25) (layer F.Cu) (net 32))
 (segment (start 142.97 89.7) (end 143.5 89.7) (width 0.25) (layer F.Cu) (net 32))
 (segment (start 144.1 89.3) (end 144.1 89.7) (width 0.25) (layer F.Cu) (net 32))
 (segment (start 144.1 88.9) (end 144.1 89.3) (width 0.25) (layer F.Cu) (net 32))
 (segment (start 144.1 88.5) (end 144.1 88.9) (width 0.25) (layer F.Cu) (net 32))
 (segment (start 142.97 89.3) (end 144.1 89.3) (width 0.25) (layer F.Cu) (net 32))
 (segment (start 142.97 88.9) (end 144.1 88.9) (width 0.25) (layer F.Cu) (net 32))
 (segment (start 142.97 88.5) (end 144.1 88.5) (width 0.25) (layer F.Cu) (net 32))
 (segment (start 136.4 89.7) (end 136.4 88.5) (width 0.25) (layer F.Cu) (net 27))
 (segment (start 136.4 88.5) (end 135.35 88.5) (width 0.25) (layer F.Cu) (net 27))
 (segment (start 135.35 88.9) (end 136.4 88.9) (width 0.25) (layer F.Cu) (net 27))
 (segment (start 135.35 89.3) (end 136.4 89.3) (width 0.25) (layer F.Cu) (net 27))
 (segment (start 135.35 90.1) (end 136.4 90.1) (width 0.25) (layer F.Cu) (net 27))
 (segment (start 136.4 89.7) (end 135.35 89.7) (width 0.25) (layer F.Cu) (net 27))
 (segment (start 136.4 90.1) (end 136.4 89.7) (width 0.25) (layer F.Cu) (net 27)))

